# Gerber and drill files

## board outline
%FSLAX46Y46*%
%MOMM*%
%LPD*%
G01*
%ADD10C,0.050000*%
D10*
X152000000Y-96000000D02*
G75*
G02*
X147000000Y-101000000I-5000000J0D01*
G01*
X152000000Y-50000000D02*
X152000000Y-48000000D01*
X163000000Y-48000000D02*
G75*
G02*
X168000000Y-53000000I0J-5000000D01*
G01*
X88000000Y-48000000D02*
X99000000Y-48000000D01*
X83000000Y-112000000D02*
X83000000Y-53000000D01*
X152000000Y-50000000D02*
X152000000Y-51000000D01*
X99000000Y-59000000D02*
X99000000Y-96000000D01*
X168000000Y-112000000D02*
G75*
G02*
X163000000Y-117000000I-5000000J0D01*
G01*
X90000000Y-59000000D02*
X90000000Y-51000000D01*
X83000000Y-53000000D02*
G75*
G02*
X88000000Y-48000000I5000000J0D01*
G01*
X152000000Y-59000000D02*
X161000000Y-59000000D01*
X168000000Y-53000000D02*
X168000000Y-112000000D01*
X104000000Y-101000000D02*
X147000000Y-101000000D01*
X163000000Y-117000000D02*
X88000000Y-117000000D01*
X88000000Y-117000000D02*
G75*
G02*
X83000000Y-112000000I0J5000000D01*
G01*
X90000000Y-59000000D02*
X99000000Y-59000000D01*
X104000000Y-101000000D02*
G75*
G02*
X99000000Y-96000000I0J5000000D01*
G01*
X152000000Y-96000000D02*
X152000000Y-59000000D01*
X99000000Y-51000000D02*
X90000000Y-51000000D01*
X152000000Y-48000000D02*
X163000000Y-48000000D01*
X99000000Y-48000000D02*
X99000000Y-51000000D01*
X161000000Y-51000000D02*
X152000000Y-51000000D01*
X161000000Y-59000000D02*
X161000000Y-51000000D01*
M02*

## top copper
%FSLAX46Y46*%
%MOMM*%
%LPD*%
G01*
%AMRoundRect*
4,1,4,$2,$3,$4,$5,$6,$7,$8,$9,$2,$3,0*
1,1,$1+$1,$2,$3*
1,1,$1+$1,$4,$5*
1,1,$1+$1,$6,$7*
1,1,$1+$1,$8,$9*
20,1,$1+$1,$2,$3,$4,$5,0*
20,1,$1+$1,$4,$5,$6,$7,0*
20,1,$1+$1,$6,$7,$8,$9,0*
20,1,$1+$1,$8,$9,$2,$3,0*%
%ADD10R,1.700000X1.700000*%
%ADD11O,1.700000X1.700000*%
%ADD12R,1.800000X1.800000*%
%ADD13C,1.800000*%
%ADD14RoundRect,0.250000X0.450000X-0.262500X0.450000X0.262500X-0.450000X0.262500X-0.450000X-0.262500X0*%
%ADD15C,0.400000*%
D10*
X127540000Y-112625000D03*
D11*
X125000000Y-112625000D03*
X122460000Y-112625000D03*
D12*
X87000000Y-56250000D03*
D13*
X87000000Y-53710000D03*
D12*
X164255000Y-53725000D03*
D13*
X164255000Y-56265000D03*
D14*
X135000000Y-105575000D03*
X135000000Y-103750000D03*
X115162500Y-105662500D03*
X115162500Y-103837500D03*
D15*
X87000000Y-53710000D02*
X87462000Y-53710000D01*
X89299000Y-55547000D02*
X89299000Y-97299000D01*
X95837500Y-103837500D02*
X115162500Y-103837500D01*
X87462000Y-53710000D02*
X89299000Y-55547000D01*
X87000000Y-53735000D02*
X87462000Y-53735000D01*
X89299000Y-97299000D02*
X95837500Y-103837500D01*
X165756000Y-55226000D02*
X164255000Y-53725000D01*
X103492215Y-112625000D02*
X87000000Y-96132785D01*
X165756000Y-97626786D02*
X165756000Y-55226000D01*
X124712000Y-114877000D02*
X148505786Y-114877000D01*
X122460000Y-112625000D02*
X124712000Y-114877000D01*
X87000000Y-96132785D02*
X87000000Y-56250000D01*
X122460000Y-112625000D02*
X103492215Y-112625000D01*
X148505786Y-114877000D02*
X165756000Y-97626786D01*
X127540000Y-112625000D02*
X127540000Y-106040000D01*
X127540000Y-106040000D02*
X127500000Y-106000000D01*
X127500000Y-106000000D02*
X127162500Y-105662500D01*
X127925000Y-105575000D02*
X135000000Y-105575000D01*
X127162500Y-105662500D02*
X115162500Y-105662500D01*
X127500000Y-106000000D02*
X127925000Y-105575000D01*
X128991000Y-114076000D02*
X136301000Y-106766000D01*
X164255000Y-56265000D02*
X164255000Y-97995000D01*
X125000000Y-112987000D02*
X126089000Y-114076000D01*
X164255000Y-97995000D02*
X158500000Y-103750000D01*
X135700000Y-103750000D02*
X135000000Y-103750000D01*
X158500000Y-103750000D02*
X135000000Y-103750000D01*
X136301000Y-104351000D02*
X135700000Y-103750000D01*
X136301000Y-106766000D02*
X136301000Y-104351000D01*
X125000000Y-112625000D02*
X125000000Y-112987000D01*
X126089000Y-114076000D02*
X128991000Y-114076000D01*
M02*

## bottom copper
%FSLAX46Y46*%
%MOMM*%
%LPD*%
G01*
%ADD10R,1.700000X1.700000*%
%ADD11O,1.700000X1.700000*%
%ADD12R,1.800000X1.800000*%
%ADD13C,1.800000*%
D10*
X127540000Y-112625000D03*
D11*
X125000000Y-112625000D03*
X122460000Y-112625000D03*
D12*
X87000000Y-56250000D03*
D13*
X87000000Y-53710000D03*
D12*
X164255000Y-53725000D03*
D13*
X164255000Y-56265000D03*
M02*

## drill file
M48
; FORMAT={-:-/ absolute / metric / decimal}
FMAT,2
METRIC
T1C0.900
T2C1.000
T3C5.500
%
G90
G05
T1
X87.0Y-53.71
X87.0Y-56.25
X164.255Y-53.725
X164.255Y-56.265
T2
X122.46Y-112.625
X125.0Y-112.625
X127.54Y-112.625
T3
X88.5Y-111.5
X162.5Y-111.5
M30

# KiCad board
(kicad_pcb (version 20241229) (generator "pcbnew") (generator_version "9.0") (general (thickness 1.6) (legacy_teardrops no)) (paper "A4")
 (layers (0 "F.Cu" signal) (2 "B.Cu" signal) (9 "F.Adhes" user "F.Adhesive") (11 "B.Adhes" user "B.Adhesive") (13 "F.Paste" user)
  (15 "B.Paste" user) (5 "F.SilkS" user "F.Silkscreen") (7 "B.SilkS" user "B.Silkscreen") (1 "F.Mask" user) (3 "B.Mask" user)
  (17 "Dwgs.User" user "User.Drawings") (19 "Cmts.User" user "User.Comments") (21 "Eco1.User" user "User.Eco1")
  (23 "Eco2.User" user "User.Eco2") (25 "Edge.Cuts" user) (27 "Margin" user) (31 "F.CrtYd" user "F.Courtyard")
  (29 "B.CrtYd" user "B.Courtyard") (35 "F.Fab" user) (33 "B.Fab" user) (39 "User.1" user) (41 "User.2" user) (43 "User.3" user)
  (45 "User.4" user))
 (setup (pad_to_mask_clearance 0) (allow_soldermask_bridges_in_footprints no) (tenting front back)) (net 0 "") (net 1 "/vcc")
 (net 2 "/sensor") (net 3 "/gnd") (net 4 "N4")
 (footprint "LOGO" (layer "F.Cu") (at 92.75 75.25 90)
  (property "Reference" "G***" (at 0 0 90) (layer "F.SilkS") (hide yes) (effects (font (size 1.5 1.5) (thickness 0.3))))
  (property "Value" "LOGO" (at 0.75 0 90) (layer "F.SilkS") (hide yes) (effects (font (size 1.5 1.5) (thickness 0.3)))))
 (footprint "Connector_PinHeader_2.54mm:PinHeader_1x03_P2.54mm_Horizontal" (layer "F.Cu") (at 127.54 112.625 -90)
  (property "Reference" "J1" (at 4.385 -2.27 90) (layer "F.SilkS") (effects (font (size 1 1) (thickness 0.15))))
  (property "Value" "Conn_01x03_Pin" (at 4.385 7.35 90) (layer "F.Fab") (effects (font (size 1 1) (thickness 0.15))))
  (pad "1" thru_hole rect (at 0 0 270) (size 1.7 1.7) (drill 1) (layers "*.Cu" "*.Mask") (remove_unused_layers no) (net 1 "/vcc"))
  (pad "2" thru_hole oval (at 0 2.54 270) (size 1.7 1.7) (drill 1) (layers "*.Cu" "*.Mask") (remove_unused_layers no) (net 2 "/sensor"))
  (pad "3" thru_hole oval (at 0 5.08 270) (size 1.7 1.7) (drill 1) (layers "*.Cu" "*.Mask") (remove_unused_layers no) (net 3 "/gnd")))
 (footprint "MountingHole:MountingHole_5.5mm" (layer "F.Cu") (at 88.5 111.5)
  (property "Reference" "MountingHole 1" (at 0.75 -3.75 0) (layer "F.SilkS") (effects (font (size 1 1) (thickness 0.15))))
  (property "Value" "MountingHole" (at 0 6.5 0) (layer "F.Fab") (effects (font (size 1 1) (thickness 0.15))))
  (pad "" np_thru_hole circle (at 0 0) (size 5.5 5.5) (drill 5.5) (layers "*.Cu" "*.Mask")))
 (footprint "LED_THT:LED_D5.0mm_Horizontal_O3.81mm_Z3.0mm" (layer "F.Cu") (at 87 56.25 90)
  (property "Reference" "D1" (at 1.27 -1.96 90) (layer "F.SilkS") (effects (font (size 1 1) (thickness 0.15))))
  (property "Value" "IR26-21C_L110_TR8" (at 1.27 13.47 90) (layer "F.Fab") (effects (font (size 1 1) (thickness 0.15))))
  (pad "1" thru_hole rect (at 0 0 90) (size 1.8 1.8) (drill 0.9) (layers "*.Cu" "*.Mask") (remove_unused_layers no) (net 3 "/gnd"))
  (pad "2" thru_hole circle (at 2.54 0 90) (size 1.8 1.8) (drill 0.9) (layers "*.Cu" "*.Mask") (remove_unused_layers no) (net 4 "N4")))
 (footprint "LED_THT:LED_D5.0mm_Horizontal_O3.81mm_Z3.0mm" (layer "F.Cu") (at 164.255 53.725 -90)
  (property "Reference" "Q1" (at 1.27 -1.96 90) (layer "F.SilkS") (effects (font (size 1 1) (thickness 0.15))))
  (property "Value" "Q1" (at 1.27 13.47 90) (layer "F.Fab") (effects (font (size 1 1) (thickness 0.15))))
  (pad "1" thru_hole rect (at 0 0 270) (size 1.8 1.8) (drill 0.9) (layers "*.Cu" "*.Mask") (remove_unused_layers no) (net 3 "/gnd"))
  (pad "2" thru_hole circle (at 2.54 0 270) (size 1.8 1.8) (drill 0.9) (layers "*.Cu" "*.Mask") (remove_unused_layers no) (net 2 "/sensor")))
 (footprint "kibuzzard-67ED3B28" (layer "F.Cu") (at 159.75 80.25 -90)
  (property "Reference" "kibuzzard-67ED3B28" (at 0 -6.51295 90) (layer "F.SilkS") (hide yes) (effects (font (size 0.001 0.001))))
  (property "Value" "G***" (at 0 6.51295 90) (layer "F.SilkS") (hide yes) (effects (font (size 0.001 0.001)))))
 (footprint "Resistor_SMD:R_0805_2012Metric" (layer "F.Cu") (at 135 104.6625 90)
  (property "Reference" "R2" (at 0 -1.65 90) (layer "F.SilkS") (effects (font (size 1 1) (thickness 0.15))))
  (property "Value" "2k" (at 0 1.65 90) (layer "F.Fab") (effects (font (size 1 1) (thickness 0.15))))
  (pad "1" smd roundrect (at -0.9125 0 90) (size 1.025 1.4) (layers "F.Cu" "F.Mask" "F.Paste") (roundrect_rratio 0.243902) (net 1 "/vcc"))
  (pad "2" smd roundrect (at 0.9125 0 90) (size 1.025 1.4) (layers "F.Cu" "F.Mask" "F.Paste") (roundrect_rratio 0.243902) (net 2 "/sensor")))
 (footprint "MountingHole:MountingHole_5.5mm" (layer "F.Cu") (at 162.5 111.5)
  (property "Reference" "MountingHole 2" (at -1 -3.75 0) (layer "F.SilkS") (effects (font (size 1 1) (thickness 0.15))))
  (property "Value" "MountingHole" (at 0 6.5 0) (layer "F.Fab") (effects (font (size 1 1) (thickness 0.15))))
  (pad "" np_thru_hole circle (at 0 0) (size 5.5 5.5) (drill 5.5) (layers "*.Cu" "*.Mask")))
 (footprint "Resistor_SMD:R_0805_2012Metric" (layer "F.Cu") (at 115.1625 104.75 90)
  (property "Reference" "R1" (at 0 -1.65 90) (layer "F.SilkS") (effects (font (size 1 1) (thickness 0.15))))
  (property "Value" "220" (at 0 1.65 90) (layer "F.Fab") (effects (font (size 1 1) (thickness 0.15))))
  (pad "1" smd roundrect (at -0.9125 0 90) (size 1.025 1.4) (layers "F.Cu" "F.Mask" "F.Paste") (roundrect_rratio 0.243902) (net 1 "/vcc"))
  (pad "2" smd roundrect (at 0.9125 0 90) (size 1.025 1.4) (layers "F.Cu" "F.Mask" "F.Paste") (roundrect_rratio 0.243902) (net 4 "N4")))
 (gr_arc (start 152 96) (mid 150.535534 99.535534) (end 147 101) (stroke (width 0.05) (type default)) (layer "Edge.Cuts"))
 (gr_line (start 152 50) (end 152 48) (stroke (width 0.05) (type default)) (layer "Edge.Cuts"))
 (gr_arc (start 163 48) (mid 166.535534 49.464466) (end 168 53) (stroke (width 0.05) (type default)) (layer "Edge.Cuts"))
 (gr_line (start 88 48) (end 99 48) (stroke (width 0.05) (type default)) (layer "Edge.Cuts"))
 (gr_line (start 83 112) (end 83 53) (stroke (width 0.05) (type default)) (layer "Edge.Cuts"))
 (gr_line (start 152 50) (end 152 51) (stroke (width 0.05) (type default)) (layer "Edge.Cuts"))
 (gr_line (start 99 59) (end 99 96) (stroke (width 0.05) (type default)) (layer "Edge.Cuts"))
 (gr_arc (start 168 112) (mid 166.535534 115.535534) (end 163 117) (stroke (width 0.05) (type default)) (layer "Edge.Cuts"))
 (gr_line (start 90 59) (end 90 51) (stroke (width 0.05) (type default)) (layer "Edge.Cuts"))
 (gr_arc (start 83 53) (mid 84.464466 49.464466) (end 88 48) (stroke (width 0.05) (type default)) (layer "Edge.Cuts"))
 (gr_line (start 152 59) (end 161 59) (stroke (width 0.05) (type default)) (layer "Edge.Cuts"))
 (gr_line (start 168 53) (end 168 112) (stroke (width 0.05) (type default)) (layer "Edge.Cuts"))
 (gr_line (start 104 101) (end 147 101) (stroke (width 0.05) (type default)) (layer "Edge.Cuts"))
 (gr_line (start 163 117) (end 88 117) (stroke (width 0.05) (type default)) (layer "Edge.Cuts"))
 (gr_arc (start 88 117) (mid 84.464466 115.535534) (end 83 112) (stroke (width 0.05) (type default)) (layer "Edge.Cuts"))
 (gr_line (start 90 59) (end 99 59) (stroke (width 0.05) (type default)) (layer "Edge.Cuts"))
 (gr_arc (start 104 101) (mid 100.464466 99.535534) (end 99 96) (stroke (width 0.05) (type default)) (layer "Edge.Cuts"))
 (gr_line (start 152 96) (end 152 59) (stroke (width 0.05) (type default)) (layer "Edge.Cuts"))
 (gr_line (start 99 51) (end 90 51) (stroke (width 0.05) (type default)) (layer "Edge.Cuts"))
 (gr_line (start 152 48) (end 163 48) (stroke (width 0.05) (type default)) (layer "Edge.Cuts"))
 (gr_line (start 99 48) (end 99 51) (stroke (width 0.05) (type default)) (layer "Edge.Cuts"))
 (gr_line (start 161 51) (end 152 51) (stroke (width 0.05) (type default)) (layer "Edge.Cuts"))
 (gr_line (start 161 59) (end 161 51) (stroke (width 0.05) (type default)) (layer "Edge.Cuts"))
 (segment (start 87 53.71) (end 87.462 53.71) (width 0.4) (layer "F.Cu") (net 4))
 (segment (start 89.299 55.547) (end 89.299 97.299) (width 0.4) (layer "F.Cu") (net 4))
 (segment (start 95.8375 103.8375) (end 115.1625 103.8375) (width 0.4) (layer "F.Cu") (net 4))
 (segment (start 87.462 53.71) (end 89.299 55.547) (width 0.4) (layer "F.Cu") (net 4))
 (segment (start 87 53.735) (end 87.462 53.735) (width 0.4) (layer "F.Cu") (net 4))
 (segment (start 89.299 97.299) (end 95.8375 103.8375) (width 0.4) (layer "F.Cu") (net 4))
 (segment (start 165.756 55.226) (end 164.255 53.725) (width 0.4) (layer "F.Cu") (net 3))
 (segment (start 103.492215 112.625) (end 87 96.132785) (width 0.4) (layer "F.Cu") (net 3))
 (segment (start 165.756 97.626786) (end 165.756 55.226) (width 0.4) (layer "F.Cu") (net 3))
 (segment (start 124.712 114.877) (end 148.505786 114.877) (width 0.4) (layer "F.Cu") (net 3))
 (segment (start 122.46 112.625) (end 124.712 114.877) (width 0.4) (layer "F.Cu") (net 3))
 (segment (start 87 96.132785) (end 87 56.25) (width 0.4) (layer "F.Cu") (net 3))
 (segment (start 122.46 112.625) (end 103.492215 112.625) (width 0.4) (layer "F.Cu") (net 3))
 (segment (start 148.505786 114.877) (end 165.756 97.626786) (width 0.4) (layer "F.Cu") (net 3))
 (segment (start 127.54 112.625) (end 127.54 106.04) (width 0.4) (layer "F.Cu") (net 1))
 (segment (start 127.54 106.04) (end 127.5 106) (width 0.4) (layer "F.Cu") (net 1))
 (segment (start 127.5 106) (end 127.1625 105.6625) (width 0.4) (layer "F.Cu") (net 1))
 (segment (start 127.925 105.575) (end 135 105.575) (width 0.4) (layer "F.Cu") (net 1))
 (segment (start 127.1625 105.6625) (end 115.1625 105.6625) (width 0.4) (layer "F.Cu") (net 1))
 (segment (start 127.5 106) (end 127.925 105.575) (width 0.4) (layer "F.Cu") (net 1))
 (segment (start 128.991 114.076) (end 136.301 106.766) (width 0.4) (layer "F.Cu") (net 2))
 (segment (start 164.255 56.265) (end 164.255 97.995) (width 0.4) (layer "F.Cu") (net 2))
 (segment (start 125 112.987) (end 126.089 114.076) (width 0.4) (layer "F.Cu") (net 2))
 (segment (start 164.255 97.995) (end 158.5 103.75) (width 0.4) (layer "F.Cu") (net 2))
 (segment (start 135.7 103.75) (end 135 103.75) (width 0.4) (layer "F.Cu") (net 2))
 (segment (start 158.5 103.75) (end 135 103.75) (width 0.4) (layer "F.Cu") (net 2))
 (segment (start 136.301 104.351) (end 135.7 103.75) (width 0.4) (layer "F.Cu") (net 2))
 (segment (start 136.301 106.766) (end 136.301 104.351) (width 0.4) (layer "F.Cu") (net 2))
 (segment (start 125 112.625) (end 125 112.987) (width 0.4) (layer "F.Cu") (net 2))
 (segment (start 126.089 114.076) (end 128.991 114.076) (width 0.4) (layer "F.Cu") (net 2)))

